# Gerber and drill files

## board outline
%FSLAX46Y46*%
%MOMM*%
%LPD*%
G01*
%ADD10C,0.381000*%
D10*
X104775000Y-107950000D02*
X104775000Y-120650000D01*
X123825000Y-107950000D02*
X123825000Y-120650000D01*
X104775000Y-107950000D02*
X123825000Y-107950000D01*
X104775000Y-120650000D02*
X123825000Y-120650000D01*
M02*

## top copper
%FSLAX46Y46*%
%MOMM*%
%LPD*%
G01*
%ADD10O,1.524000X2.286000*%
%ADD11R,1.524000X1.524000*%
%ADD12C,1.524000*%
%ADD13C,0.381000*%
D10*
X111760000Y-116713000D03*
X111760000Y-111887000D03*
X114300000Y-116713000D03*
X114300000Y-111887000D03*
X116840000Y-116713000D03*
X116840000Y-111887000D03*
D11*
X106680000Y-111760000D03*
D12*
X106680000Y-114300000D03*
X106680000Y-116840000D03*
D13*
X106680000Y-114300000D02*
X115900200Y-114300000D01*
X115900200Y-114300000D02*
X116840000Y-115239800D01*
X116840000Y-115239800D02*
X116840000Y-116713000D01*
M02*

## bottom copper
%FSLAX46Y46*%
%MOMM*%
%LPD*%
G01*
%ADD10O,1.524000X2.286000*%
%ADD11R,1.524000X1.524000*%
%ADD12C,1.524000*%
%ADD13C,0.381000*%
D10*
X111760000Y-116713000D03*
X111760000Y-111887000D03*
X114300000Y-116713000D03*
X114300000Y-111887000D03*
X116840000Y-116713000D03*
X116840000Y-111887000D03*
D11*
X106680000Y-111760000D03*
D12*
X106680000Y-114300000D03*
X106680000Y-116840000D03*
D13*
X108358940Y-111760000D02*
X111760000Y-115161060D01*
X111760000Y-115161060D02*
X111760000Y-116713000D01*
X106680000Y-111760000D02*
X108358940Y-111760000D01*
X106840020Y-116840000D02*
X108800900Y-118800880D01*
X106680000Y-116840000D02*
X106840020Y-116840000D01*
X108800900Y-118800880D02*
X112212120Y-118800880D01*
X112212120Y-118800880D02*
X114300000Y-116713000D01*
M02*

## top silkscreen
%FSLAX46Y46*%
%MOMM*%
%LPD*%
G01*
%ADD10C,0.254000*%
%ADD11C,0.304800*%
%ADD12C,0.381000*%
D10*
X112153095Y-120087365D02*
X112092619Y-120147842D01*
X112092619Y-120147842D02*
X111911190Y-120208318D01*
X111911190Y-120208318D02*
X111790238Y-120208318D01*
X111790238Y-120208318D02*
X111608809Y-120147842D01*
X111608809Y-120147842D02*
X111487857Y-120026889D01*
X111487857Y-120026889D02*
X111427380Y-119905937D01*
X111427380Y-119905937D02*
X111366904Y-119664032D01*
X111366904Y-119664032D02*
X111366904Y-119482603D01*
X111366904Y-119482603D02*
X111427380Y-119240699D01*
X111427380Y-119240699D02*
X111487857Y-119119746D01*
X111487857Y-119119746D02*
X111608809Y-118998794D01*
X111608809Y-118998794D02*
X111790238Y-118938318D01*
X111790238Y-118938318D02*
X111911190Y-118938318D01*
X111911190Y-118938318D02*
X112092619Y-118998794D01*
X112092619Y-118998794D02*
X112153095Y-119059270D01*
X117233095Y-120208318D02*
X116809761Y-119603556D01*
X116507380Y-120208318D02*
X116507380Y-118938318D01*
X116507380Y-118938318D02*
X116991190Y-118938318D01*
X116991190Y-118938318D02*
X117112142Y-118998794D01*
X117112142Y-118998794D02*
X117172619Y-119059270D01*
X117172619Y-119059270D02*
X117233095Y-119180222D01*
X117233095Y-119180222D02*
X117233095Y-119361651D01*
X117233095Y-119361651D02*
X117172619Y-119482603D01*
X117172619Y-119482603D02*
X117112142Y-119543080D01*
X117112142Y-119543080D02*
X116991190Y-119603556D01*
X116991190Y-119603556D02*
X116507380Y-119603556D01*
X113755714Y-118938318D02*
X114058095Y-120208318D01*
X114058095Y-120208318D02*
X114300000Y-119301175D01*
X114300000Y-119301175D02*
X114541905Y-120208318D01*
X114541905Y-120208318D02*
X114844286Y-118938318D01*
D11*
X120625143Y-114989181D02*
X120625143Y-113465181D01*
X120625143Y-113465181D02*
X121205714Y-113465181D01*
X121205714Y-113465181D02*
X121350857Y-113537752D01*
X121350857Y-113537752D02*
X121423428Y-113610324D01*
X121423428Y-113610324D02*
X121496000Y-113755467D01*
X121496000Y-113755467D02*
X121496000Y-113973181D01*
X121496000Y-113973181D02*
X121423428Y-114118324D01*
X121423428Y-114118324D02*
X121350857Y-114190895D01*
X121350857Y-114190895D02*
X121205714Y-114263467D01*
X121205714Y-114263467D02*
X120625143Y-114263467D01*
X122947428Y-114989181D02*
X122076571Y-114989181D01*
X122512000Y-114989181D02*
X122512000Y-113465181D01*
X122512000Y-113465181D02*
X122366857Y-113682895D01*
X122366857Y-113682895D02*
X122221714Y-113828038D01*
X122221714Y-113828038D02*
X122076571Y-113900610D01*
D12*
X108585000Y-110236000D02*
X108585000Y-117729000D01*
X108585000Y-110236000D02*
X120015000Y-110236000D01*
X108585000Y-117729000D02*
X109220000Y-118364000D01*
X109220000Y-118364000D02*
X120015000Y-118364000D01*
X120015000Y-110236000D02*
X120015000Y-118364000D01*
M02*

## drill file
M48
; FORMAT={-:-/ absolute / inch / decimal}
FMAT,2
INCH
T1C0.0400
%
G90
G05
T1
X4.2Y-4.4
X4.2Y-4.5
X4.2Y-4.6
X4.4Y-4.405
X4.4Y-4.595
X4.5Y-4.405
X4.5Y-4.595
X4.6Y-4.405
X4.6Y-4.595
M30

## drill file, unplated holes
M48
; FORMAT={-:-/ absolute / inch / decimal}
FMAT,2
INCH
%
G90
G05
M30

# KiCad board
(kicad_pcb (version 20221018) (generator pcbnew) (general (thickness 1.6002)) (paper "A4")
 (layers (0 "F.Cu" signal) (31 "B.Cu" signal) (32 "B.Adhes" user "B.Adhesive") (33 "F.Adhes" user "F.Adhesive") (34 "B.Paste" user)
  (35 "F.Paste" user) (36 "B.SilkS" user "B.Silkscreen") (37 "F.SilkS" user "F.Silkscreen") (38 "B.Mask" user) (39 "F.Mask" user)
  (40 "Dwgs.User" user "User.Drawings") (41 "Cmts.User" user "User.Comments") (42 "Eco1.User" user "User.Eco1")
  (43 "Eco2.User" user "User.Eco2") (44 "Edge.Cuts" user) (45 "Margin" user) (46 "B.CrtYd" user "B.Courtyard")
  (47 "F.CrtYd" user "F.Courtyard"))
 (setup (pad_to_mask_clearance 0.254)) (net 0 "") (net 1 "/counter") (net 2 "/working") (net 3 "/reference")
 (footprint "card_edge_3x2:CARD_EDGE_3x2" (layer "F.Cu") (at 114.3 114.3)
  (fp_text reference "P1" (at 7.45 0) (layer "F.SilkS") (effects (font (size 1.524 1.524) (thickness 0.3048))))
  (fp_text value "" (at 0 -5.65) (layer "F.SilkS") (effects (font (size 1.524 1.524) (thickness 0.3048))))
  (fp_line (start -5.715 -4.064) (end -5.715 3.429) (stroke (width 0.381) (type solid)) (layer "F.SilkS"))
  (fp_line (start -5.715 -4.064) (end 5.715 -4.064) (stroke (width 0.381) (type solid)) (layer "F.SilkS"))
  (fp_line (start -5.715 3.429) (end -5.08 4.064) (stroke (width 0.381) (type solid)) (layer "F.SilkS"))
  (fp_line (start -5.08 4.064) (end 5.715 4.064) (stroke (width 0.381) (type solid)) (layer "F.SilkS"))
  (fp_line (start 5.715 -4.064) (end 5.715 4.064) (stroke (width 0.381) (type solid)) (layer "F.SilkS"))
  (pad "1" thru_hole oval (at -2.54 2.413) (size 1.524 2.286) (drill 1.016) (layers "*.Cu" "*.Mask") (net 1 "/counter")
   (thermal_bridge_angle 45))
  (pad "2" thru_hole oval (at -2.54 -2.413) (size 1.524 2.286) (drill 1.016) (layers "*.Cu" "*.Mask") (thermal_bridge_angle 45))
  (pad "3" thru_hole oval (at 0 2.413) (size 1.524 2.286) (drill 1.016) (layers "*.Cu" "*.Mask") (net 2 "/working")
   (thermal_bridge_angle 45))
  (pad "4" thru_hole oval (at 0 -2.413) (size 1.524 2.286) (drill 1.016) (layers "*.Cu" "*.Mask") (thermal_bridge_angle 45))
  (pad "5" thru_hole oval (at 2.54 2.413) (size 1.524 2.286) (drill 1.016) (layers "*.Cu" "*.Mask") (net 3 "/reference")
   (thermal_bridge_angle 45))
  (pad "6" thru_hole oval (at 2.54 -2.413) (size 1.524 2.286) (drill 1.016) (layers "*.Cu" "*.Mask") (thermal_bridge_angle 45)))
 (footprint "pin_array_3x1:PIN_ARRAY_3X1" (layer "B.Cu") (at 106.68 114.3 -90)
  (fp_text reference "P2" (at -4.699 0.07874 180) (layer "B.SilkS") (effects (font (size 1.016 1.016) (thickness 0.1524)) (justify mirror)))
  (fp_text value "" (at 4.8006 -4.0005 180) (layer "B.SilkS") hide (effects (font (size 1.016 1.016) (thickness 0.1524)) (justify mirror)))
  (pad "1" thru_hole rect (at -2.54 0 270) (size 1.524 1.524) (drill 1.016) (layers "*.Cu" "*.Mask") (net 1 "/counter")
   (thermal_bridge_angle 45))
  (pad "2" thru_hole circle (at 0 0 270) (size 1.524 1.524) (drill 1.016) (layers "*.Cu" "*.Mask") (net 3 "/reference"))
  (pad "3" thru_hole circle (at 2.54 0 270) (size 1.524 1.524) (drill 1.016) (layers "*.Cu" "*.Mask") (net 2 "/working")))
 (gr_line (start 104.775 107.95) (end 104.775 120.65) (stroke (width 0.381) (type solid)) (layer "Edge.Cuts"))
 (gr_line (start 123.825 107.95) (end 123.825 120.65) (stroke (width 0.381) (type solid)) (layer "Edge.Cuts"))
 (gr_line (start 104.775 107.95) (end 123.825 107.95) (stroke (width 0.381) (type solid)) (layer "Edge.Cuts"))
 (gr_line (start 104.775 120.65) (end 123.825 120.65) (stroke (width 0.381) (type solid)) (layer "Edge.Cuts"))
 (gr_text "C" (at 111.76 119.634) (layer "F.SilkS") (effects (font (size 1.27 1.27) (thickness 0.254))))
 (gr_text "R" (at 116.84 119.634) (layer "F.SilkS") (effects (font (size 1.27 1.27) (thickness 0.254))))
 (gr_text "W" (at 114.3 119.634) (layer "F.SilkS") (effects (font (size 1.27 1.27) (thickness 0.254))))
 (segment (start 108.35894 111.76) (end 111.76 115.16106) (width 0.381) (layer "B.Cu") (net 1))
 (segment (start 111.76 115.16106) (end 111.76 116.713) (width 0.381) (layer "B.Cu") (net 1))
 (segment (start 106.68 111.76) (end 108.35894 111.76) (width 0.381) (layer "B.Cu") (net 1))
 (segment (start 106.68 114.3) (end 115.9002 114.3) (width 0.381) (layer "F.Cu") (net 3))
 (segment (start 115.9002 114.3) (end 116.84 115.2398) (width 0.381) (layer "F.Cu") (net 3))
 (segment (start 116.84 115.2398) (end 116.84 116.713) (width 0.381) (layer "F.Cu") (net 3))
 (segment (start 106.84002 116.84) (end 108.8009 118.80088) (width 0.381) (layer "B.Cu") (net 2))
 (segment (start 106.68 116.84) (end 106.84002 116.84) (width 0.381) (layer "B.Cu") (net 2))
 (segment (start 108.8009 118.80088) (end 112.21212 118.80088) (width 0.381) (layer "B.Cu") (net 2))
 (segment (start 112.21212 118.80088) (end 114.3 116.713) (width 0.381) (layer "B.Cu") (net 2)))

